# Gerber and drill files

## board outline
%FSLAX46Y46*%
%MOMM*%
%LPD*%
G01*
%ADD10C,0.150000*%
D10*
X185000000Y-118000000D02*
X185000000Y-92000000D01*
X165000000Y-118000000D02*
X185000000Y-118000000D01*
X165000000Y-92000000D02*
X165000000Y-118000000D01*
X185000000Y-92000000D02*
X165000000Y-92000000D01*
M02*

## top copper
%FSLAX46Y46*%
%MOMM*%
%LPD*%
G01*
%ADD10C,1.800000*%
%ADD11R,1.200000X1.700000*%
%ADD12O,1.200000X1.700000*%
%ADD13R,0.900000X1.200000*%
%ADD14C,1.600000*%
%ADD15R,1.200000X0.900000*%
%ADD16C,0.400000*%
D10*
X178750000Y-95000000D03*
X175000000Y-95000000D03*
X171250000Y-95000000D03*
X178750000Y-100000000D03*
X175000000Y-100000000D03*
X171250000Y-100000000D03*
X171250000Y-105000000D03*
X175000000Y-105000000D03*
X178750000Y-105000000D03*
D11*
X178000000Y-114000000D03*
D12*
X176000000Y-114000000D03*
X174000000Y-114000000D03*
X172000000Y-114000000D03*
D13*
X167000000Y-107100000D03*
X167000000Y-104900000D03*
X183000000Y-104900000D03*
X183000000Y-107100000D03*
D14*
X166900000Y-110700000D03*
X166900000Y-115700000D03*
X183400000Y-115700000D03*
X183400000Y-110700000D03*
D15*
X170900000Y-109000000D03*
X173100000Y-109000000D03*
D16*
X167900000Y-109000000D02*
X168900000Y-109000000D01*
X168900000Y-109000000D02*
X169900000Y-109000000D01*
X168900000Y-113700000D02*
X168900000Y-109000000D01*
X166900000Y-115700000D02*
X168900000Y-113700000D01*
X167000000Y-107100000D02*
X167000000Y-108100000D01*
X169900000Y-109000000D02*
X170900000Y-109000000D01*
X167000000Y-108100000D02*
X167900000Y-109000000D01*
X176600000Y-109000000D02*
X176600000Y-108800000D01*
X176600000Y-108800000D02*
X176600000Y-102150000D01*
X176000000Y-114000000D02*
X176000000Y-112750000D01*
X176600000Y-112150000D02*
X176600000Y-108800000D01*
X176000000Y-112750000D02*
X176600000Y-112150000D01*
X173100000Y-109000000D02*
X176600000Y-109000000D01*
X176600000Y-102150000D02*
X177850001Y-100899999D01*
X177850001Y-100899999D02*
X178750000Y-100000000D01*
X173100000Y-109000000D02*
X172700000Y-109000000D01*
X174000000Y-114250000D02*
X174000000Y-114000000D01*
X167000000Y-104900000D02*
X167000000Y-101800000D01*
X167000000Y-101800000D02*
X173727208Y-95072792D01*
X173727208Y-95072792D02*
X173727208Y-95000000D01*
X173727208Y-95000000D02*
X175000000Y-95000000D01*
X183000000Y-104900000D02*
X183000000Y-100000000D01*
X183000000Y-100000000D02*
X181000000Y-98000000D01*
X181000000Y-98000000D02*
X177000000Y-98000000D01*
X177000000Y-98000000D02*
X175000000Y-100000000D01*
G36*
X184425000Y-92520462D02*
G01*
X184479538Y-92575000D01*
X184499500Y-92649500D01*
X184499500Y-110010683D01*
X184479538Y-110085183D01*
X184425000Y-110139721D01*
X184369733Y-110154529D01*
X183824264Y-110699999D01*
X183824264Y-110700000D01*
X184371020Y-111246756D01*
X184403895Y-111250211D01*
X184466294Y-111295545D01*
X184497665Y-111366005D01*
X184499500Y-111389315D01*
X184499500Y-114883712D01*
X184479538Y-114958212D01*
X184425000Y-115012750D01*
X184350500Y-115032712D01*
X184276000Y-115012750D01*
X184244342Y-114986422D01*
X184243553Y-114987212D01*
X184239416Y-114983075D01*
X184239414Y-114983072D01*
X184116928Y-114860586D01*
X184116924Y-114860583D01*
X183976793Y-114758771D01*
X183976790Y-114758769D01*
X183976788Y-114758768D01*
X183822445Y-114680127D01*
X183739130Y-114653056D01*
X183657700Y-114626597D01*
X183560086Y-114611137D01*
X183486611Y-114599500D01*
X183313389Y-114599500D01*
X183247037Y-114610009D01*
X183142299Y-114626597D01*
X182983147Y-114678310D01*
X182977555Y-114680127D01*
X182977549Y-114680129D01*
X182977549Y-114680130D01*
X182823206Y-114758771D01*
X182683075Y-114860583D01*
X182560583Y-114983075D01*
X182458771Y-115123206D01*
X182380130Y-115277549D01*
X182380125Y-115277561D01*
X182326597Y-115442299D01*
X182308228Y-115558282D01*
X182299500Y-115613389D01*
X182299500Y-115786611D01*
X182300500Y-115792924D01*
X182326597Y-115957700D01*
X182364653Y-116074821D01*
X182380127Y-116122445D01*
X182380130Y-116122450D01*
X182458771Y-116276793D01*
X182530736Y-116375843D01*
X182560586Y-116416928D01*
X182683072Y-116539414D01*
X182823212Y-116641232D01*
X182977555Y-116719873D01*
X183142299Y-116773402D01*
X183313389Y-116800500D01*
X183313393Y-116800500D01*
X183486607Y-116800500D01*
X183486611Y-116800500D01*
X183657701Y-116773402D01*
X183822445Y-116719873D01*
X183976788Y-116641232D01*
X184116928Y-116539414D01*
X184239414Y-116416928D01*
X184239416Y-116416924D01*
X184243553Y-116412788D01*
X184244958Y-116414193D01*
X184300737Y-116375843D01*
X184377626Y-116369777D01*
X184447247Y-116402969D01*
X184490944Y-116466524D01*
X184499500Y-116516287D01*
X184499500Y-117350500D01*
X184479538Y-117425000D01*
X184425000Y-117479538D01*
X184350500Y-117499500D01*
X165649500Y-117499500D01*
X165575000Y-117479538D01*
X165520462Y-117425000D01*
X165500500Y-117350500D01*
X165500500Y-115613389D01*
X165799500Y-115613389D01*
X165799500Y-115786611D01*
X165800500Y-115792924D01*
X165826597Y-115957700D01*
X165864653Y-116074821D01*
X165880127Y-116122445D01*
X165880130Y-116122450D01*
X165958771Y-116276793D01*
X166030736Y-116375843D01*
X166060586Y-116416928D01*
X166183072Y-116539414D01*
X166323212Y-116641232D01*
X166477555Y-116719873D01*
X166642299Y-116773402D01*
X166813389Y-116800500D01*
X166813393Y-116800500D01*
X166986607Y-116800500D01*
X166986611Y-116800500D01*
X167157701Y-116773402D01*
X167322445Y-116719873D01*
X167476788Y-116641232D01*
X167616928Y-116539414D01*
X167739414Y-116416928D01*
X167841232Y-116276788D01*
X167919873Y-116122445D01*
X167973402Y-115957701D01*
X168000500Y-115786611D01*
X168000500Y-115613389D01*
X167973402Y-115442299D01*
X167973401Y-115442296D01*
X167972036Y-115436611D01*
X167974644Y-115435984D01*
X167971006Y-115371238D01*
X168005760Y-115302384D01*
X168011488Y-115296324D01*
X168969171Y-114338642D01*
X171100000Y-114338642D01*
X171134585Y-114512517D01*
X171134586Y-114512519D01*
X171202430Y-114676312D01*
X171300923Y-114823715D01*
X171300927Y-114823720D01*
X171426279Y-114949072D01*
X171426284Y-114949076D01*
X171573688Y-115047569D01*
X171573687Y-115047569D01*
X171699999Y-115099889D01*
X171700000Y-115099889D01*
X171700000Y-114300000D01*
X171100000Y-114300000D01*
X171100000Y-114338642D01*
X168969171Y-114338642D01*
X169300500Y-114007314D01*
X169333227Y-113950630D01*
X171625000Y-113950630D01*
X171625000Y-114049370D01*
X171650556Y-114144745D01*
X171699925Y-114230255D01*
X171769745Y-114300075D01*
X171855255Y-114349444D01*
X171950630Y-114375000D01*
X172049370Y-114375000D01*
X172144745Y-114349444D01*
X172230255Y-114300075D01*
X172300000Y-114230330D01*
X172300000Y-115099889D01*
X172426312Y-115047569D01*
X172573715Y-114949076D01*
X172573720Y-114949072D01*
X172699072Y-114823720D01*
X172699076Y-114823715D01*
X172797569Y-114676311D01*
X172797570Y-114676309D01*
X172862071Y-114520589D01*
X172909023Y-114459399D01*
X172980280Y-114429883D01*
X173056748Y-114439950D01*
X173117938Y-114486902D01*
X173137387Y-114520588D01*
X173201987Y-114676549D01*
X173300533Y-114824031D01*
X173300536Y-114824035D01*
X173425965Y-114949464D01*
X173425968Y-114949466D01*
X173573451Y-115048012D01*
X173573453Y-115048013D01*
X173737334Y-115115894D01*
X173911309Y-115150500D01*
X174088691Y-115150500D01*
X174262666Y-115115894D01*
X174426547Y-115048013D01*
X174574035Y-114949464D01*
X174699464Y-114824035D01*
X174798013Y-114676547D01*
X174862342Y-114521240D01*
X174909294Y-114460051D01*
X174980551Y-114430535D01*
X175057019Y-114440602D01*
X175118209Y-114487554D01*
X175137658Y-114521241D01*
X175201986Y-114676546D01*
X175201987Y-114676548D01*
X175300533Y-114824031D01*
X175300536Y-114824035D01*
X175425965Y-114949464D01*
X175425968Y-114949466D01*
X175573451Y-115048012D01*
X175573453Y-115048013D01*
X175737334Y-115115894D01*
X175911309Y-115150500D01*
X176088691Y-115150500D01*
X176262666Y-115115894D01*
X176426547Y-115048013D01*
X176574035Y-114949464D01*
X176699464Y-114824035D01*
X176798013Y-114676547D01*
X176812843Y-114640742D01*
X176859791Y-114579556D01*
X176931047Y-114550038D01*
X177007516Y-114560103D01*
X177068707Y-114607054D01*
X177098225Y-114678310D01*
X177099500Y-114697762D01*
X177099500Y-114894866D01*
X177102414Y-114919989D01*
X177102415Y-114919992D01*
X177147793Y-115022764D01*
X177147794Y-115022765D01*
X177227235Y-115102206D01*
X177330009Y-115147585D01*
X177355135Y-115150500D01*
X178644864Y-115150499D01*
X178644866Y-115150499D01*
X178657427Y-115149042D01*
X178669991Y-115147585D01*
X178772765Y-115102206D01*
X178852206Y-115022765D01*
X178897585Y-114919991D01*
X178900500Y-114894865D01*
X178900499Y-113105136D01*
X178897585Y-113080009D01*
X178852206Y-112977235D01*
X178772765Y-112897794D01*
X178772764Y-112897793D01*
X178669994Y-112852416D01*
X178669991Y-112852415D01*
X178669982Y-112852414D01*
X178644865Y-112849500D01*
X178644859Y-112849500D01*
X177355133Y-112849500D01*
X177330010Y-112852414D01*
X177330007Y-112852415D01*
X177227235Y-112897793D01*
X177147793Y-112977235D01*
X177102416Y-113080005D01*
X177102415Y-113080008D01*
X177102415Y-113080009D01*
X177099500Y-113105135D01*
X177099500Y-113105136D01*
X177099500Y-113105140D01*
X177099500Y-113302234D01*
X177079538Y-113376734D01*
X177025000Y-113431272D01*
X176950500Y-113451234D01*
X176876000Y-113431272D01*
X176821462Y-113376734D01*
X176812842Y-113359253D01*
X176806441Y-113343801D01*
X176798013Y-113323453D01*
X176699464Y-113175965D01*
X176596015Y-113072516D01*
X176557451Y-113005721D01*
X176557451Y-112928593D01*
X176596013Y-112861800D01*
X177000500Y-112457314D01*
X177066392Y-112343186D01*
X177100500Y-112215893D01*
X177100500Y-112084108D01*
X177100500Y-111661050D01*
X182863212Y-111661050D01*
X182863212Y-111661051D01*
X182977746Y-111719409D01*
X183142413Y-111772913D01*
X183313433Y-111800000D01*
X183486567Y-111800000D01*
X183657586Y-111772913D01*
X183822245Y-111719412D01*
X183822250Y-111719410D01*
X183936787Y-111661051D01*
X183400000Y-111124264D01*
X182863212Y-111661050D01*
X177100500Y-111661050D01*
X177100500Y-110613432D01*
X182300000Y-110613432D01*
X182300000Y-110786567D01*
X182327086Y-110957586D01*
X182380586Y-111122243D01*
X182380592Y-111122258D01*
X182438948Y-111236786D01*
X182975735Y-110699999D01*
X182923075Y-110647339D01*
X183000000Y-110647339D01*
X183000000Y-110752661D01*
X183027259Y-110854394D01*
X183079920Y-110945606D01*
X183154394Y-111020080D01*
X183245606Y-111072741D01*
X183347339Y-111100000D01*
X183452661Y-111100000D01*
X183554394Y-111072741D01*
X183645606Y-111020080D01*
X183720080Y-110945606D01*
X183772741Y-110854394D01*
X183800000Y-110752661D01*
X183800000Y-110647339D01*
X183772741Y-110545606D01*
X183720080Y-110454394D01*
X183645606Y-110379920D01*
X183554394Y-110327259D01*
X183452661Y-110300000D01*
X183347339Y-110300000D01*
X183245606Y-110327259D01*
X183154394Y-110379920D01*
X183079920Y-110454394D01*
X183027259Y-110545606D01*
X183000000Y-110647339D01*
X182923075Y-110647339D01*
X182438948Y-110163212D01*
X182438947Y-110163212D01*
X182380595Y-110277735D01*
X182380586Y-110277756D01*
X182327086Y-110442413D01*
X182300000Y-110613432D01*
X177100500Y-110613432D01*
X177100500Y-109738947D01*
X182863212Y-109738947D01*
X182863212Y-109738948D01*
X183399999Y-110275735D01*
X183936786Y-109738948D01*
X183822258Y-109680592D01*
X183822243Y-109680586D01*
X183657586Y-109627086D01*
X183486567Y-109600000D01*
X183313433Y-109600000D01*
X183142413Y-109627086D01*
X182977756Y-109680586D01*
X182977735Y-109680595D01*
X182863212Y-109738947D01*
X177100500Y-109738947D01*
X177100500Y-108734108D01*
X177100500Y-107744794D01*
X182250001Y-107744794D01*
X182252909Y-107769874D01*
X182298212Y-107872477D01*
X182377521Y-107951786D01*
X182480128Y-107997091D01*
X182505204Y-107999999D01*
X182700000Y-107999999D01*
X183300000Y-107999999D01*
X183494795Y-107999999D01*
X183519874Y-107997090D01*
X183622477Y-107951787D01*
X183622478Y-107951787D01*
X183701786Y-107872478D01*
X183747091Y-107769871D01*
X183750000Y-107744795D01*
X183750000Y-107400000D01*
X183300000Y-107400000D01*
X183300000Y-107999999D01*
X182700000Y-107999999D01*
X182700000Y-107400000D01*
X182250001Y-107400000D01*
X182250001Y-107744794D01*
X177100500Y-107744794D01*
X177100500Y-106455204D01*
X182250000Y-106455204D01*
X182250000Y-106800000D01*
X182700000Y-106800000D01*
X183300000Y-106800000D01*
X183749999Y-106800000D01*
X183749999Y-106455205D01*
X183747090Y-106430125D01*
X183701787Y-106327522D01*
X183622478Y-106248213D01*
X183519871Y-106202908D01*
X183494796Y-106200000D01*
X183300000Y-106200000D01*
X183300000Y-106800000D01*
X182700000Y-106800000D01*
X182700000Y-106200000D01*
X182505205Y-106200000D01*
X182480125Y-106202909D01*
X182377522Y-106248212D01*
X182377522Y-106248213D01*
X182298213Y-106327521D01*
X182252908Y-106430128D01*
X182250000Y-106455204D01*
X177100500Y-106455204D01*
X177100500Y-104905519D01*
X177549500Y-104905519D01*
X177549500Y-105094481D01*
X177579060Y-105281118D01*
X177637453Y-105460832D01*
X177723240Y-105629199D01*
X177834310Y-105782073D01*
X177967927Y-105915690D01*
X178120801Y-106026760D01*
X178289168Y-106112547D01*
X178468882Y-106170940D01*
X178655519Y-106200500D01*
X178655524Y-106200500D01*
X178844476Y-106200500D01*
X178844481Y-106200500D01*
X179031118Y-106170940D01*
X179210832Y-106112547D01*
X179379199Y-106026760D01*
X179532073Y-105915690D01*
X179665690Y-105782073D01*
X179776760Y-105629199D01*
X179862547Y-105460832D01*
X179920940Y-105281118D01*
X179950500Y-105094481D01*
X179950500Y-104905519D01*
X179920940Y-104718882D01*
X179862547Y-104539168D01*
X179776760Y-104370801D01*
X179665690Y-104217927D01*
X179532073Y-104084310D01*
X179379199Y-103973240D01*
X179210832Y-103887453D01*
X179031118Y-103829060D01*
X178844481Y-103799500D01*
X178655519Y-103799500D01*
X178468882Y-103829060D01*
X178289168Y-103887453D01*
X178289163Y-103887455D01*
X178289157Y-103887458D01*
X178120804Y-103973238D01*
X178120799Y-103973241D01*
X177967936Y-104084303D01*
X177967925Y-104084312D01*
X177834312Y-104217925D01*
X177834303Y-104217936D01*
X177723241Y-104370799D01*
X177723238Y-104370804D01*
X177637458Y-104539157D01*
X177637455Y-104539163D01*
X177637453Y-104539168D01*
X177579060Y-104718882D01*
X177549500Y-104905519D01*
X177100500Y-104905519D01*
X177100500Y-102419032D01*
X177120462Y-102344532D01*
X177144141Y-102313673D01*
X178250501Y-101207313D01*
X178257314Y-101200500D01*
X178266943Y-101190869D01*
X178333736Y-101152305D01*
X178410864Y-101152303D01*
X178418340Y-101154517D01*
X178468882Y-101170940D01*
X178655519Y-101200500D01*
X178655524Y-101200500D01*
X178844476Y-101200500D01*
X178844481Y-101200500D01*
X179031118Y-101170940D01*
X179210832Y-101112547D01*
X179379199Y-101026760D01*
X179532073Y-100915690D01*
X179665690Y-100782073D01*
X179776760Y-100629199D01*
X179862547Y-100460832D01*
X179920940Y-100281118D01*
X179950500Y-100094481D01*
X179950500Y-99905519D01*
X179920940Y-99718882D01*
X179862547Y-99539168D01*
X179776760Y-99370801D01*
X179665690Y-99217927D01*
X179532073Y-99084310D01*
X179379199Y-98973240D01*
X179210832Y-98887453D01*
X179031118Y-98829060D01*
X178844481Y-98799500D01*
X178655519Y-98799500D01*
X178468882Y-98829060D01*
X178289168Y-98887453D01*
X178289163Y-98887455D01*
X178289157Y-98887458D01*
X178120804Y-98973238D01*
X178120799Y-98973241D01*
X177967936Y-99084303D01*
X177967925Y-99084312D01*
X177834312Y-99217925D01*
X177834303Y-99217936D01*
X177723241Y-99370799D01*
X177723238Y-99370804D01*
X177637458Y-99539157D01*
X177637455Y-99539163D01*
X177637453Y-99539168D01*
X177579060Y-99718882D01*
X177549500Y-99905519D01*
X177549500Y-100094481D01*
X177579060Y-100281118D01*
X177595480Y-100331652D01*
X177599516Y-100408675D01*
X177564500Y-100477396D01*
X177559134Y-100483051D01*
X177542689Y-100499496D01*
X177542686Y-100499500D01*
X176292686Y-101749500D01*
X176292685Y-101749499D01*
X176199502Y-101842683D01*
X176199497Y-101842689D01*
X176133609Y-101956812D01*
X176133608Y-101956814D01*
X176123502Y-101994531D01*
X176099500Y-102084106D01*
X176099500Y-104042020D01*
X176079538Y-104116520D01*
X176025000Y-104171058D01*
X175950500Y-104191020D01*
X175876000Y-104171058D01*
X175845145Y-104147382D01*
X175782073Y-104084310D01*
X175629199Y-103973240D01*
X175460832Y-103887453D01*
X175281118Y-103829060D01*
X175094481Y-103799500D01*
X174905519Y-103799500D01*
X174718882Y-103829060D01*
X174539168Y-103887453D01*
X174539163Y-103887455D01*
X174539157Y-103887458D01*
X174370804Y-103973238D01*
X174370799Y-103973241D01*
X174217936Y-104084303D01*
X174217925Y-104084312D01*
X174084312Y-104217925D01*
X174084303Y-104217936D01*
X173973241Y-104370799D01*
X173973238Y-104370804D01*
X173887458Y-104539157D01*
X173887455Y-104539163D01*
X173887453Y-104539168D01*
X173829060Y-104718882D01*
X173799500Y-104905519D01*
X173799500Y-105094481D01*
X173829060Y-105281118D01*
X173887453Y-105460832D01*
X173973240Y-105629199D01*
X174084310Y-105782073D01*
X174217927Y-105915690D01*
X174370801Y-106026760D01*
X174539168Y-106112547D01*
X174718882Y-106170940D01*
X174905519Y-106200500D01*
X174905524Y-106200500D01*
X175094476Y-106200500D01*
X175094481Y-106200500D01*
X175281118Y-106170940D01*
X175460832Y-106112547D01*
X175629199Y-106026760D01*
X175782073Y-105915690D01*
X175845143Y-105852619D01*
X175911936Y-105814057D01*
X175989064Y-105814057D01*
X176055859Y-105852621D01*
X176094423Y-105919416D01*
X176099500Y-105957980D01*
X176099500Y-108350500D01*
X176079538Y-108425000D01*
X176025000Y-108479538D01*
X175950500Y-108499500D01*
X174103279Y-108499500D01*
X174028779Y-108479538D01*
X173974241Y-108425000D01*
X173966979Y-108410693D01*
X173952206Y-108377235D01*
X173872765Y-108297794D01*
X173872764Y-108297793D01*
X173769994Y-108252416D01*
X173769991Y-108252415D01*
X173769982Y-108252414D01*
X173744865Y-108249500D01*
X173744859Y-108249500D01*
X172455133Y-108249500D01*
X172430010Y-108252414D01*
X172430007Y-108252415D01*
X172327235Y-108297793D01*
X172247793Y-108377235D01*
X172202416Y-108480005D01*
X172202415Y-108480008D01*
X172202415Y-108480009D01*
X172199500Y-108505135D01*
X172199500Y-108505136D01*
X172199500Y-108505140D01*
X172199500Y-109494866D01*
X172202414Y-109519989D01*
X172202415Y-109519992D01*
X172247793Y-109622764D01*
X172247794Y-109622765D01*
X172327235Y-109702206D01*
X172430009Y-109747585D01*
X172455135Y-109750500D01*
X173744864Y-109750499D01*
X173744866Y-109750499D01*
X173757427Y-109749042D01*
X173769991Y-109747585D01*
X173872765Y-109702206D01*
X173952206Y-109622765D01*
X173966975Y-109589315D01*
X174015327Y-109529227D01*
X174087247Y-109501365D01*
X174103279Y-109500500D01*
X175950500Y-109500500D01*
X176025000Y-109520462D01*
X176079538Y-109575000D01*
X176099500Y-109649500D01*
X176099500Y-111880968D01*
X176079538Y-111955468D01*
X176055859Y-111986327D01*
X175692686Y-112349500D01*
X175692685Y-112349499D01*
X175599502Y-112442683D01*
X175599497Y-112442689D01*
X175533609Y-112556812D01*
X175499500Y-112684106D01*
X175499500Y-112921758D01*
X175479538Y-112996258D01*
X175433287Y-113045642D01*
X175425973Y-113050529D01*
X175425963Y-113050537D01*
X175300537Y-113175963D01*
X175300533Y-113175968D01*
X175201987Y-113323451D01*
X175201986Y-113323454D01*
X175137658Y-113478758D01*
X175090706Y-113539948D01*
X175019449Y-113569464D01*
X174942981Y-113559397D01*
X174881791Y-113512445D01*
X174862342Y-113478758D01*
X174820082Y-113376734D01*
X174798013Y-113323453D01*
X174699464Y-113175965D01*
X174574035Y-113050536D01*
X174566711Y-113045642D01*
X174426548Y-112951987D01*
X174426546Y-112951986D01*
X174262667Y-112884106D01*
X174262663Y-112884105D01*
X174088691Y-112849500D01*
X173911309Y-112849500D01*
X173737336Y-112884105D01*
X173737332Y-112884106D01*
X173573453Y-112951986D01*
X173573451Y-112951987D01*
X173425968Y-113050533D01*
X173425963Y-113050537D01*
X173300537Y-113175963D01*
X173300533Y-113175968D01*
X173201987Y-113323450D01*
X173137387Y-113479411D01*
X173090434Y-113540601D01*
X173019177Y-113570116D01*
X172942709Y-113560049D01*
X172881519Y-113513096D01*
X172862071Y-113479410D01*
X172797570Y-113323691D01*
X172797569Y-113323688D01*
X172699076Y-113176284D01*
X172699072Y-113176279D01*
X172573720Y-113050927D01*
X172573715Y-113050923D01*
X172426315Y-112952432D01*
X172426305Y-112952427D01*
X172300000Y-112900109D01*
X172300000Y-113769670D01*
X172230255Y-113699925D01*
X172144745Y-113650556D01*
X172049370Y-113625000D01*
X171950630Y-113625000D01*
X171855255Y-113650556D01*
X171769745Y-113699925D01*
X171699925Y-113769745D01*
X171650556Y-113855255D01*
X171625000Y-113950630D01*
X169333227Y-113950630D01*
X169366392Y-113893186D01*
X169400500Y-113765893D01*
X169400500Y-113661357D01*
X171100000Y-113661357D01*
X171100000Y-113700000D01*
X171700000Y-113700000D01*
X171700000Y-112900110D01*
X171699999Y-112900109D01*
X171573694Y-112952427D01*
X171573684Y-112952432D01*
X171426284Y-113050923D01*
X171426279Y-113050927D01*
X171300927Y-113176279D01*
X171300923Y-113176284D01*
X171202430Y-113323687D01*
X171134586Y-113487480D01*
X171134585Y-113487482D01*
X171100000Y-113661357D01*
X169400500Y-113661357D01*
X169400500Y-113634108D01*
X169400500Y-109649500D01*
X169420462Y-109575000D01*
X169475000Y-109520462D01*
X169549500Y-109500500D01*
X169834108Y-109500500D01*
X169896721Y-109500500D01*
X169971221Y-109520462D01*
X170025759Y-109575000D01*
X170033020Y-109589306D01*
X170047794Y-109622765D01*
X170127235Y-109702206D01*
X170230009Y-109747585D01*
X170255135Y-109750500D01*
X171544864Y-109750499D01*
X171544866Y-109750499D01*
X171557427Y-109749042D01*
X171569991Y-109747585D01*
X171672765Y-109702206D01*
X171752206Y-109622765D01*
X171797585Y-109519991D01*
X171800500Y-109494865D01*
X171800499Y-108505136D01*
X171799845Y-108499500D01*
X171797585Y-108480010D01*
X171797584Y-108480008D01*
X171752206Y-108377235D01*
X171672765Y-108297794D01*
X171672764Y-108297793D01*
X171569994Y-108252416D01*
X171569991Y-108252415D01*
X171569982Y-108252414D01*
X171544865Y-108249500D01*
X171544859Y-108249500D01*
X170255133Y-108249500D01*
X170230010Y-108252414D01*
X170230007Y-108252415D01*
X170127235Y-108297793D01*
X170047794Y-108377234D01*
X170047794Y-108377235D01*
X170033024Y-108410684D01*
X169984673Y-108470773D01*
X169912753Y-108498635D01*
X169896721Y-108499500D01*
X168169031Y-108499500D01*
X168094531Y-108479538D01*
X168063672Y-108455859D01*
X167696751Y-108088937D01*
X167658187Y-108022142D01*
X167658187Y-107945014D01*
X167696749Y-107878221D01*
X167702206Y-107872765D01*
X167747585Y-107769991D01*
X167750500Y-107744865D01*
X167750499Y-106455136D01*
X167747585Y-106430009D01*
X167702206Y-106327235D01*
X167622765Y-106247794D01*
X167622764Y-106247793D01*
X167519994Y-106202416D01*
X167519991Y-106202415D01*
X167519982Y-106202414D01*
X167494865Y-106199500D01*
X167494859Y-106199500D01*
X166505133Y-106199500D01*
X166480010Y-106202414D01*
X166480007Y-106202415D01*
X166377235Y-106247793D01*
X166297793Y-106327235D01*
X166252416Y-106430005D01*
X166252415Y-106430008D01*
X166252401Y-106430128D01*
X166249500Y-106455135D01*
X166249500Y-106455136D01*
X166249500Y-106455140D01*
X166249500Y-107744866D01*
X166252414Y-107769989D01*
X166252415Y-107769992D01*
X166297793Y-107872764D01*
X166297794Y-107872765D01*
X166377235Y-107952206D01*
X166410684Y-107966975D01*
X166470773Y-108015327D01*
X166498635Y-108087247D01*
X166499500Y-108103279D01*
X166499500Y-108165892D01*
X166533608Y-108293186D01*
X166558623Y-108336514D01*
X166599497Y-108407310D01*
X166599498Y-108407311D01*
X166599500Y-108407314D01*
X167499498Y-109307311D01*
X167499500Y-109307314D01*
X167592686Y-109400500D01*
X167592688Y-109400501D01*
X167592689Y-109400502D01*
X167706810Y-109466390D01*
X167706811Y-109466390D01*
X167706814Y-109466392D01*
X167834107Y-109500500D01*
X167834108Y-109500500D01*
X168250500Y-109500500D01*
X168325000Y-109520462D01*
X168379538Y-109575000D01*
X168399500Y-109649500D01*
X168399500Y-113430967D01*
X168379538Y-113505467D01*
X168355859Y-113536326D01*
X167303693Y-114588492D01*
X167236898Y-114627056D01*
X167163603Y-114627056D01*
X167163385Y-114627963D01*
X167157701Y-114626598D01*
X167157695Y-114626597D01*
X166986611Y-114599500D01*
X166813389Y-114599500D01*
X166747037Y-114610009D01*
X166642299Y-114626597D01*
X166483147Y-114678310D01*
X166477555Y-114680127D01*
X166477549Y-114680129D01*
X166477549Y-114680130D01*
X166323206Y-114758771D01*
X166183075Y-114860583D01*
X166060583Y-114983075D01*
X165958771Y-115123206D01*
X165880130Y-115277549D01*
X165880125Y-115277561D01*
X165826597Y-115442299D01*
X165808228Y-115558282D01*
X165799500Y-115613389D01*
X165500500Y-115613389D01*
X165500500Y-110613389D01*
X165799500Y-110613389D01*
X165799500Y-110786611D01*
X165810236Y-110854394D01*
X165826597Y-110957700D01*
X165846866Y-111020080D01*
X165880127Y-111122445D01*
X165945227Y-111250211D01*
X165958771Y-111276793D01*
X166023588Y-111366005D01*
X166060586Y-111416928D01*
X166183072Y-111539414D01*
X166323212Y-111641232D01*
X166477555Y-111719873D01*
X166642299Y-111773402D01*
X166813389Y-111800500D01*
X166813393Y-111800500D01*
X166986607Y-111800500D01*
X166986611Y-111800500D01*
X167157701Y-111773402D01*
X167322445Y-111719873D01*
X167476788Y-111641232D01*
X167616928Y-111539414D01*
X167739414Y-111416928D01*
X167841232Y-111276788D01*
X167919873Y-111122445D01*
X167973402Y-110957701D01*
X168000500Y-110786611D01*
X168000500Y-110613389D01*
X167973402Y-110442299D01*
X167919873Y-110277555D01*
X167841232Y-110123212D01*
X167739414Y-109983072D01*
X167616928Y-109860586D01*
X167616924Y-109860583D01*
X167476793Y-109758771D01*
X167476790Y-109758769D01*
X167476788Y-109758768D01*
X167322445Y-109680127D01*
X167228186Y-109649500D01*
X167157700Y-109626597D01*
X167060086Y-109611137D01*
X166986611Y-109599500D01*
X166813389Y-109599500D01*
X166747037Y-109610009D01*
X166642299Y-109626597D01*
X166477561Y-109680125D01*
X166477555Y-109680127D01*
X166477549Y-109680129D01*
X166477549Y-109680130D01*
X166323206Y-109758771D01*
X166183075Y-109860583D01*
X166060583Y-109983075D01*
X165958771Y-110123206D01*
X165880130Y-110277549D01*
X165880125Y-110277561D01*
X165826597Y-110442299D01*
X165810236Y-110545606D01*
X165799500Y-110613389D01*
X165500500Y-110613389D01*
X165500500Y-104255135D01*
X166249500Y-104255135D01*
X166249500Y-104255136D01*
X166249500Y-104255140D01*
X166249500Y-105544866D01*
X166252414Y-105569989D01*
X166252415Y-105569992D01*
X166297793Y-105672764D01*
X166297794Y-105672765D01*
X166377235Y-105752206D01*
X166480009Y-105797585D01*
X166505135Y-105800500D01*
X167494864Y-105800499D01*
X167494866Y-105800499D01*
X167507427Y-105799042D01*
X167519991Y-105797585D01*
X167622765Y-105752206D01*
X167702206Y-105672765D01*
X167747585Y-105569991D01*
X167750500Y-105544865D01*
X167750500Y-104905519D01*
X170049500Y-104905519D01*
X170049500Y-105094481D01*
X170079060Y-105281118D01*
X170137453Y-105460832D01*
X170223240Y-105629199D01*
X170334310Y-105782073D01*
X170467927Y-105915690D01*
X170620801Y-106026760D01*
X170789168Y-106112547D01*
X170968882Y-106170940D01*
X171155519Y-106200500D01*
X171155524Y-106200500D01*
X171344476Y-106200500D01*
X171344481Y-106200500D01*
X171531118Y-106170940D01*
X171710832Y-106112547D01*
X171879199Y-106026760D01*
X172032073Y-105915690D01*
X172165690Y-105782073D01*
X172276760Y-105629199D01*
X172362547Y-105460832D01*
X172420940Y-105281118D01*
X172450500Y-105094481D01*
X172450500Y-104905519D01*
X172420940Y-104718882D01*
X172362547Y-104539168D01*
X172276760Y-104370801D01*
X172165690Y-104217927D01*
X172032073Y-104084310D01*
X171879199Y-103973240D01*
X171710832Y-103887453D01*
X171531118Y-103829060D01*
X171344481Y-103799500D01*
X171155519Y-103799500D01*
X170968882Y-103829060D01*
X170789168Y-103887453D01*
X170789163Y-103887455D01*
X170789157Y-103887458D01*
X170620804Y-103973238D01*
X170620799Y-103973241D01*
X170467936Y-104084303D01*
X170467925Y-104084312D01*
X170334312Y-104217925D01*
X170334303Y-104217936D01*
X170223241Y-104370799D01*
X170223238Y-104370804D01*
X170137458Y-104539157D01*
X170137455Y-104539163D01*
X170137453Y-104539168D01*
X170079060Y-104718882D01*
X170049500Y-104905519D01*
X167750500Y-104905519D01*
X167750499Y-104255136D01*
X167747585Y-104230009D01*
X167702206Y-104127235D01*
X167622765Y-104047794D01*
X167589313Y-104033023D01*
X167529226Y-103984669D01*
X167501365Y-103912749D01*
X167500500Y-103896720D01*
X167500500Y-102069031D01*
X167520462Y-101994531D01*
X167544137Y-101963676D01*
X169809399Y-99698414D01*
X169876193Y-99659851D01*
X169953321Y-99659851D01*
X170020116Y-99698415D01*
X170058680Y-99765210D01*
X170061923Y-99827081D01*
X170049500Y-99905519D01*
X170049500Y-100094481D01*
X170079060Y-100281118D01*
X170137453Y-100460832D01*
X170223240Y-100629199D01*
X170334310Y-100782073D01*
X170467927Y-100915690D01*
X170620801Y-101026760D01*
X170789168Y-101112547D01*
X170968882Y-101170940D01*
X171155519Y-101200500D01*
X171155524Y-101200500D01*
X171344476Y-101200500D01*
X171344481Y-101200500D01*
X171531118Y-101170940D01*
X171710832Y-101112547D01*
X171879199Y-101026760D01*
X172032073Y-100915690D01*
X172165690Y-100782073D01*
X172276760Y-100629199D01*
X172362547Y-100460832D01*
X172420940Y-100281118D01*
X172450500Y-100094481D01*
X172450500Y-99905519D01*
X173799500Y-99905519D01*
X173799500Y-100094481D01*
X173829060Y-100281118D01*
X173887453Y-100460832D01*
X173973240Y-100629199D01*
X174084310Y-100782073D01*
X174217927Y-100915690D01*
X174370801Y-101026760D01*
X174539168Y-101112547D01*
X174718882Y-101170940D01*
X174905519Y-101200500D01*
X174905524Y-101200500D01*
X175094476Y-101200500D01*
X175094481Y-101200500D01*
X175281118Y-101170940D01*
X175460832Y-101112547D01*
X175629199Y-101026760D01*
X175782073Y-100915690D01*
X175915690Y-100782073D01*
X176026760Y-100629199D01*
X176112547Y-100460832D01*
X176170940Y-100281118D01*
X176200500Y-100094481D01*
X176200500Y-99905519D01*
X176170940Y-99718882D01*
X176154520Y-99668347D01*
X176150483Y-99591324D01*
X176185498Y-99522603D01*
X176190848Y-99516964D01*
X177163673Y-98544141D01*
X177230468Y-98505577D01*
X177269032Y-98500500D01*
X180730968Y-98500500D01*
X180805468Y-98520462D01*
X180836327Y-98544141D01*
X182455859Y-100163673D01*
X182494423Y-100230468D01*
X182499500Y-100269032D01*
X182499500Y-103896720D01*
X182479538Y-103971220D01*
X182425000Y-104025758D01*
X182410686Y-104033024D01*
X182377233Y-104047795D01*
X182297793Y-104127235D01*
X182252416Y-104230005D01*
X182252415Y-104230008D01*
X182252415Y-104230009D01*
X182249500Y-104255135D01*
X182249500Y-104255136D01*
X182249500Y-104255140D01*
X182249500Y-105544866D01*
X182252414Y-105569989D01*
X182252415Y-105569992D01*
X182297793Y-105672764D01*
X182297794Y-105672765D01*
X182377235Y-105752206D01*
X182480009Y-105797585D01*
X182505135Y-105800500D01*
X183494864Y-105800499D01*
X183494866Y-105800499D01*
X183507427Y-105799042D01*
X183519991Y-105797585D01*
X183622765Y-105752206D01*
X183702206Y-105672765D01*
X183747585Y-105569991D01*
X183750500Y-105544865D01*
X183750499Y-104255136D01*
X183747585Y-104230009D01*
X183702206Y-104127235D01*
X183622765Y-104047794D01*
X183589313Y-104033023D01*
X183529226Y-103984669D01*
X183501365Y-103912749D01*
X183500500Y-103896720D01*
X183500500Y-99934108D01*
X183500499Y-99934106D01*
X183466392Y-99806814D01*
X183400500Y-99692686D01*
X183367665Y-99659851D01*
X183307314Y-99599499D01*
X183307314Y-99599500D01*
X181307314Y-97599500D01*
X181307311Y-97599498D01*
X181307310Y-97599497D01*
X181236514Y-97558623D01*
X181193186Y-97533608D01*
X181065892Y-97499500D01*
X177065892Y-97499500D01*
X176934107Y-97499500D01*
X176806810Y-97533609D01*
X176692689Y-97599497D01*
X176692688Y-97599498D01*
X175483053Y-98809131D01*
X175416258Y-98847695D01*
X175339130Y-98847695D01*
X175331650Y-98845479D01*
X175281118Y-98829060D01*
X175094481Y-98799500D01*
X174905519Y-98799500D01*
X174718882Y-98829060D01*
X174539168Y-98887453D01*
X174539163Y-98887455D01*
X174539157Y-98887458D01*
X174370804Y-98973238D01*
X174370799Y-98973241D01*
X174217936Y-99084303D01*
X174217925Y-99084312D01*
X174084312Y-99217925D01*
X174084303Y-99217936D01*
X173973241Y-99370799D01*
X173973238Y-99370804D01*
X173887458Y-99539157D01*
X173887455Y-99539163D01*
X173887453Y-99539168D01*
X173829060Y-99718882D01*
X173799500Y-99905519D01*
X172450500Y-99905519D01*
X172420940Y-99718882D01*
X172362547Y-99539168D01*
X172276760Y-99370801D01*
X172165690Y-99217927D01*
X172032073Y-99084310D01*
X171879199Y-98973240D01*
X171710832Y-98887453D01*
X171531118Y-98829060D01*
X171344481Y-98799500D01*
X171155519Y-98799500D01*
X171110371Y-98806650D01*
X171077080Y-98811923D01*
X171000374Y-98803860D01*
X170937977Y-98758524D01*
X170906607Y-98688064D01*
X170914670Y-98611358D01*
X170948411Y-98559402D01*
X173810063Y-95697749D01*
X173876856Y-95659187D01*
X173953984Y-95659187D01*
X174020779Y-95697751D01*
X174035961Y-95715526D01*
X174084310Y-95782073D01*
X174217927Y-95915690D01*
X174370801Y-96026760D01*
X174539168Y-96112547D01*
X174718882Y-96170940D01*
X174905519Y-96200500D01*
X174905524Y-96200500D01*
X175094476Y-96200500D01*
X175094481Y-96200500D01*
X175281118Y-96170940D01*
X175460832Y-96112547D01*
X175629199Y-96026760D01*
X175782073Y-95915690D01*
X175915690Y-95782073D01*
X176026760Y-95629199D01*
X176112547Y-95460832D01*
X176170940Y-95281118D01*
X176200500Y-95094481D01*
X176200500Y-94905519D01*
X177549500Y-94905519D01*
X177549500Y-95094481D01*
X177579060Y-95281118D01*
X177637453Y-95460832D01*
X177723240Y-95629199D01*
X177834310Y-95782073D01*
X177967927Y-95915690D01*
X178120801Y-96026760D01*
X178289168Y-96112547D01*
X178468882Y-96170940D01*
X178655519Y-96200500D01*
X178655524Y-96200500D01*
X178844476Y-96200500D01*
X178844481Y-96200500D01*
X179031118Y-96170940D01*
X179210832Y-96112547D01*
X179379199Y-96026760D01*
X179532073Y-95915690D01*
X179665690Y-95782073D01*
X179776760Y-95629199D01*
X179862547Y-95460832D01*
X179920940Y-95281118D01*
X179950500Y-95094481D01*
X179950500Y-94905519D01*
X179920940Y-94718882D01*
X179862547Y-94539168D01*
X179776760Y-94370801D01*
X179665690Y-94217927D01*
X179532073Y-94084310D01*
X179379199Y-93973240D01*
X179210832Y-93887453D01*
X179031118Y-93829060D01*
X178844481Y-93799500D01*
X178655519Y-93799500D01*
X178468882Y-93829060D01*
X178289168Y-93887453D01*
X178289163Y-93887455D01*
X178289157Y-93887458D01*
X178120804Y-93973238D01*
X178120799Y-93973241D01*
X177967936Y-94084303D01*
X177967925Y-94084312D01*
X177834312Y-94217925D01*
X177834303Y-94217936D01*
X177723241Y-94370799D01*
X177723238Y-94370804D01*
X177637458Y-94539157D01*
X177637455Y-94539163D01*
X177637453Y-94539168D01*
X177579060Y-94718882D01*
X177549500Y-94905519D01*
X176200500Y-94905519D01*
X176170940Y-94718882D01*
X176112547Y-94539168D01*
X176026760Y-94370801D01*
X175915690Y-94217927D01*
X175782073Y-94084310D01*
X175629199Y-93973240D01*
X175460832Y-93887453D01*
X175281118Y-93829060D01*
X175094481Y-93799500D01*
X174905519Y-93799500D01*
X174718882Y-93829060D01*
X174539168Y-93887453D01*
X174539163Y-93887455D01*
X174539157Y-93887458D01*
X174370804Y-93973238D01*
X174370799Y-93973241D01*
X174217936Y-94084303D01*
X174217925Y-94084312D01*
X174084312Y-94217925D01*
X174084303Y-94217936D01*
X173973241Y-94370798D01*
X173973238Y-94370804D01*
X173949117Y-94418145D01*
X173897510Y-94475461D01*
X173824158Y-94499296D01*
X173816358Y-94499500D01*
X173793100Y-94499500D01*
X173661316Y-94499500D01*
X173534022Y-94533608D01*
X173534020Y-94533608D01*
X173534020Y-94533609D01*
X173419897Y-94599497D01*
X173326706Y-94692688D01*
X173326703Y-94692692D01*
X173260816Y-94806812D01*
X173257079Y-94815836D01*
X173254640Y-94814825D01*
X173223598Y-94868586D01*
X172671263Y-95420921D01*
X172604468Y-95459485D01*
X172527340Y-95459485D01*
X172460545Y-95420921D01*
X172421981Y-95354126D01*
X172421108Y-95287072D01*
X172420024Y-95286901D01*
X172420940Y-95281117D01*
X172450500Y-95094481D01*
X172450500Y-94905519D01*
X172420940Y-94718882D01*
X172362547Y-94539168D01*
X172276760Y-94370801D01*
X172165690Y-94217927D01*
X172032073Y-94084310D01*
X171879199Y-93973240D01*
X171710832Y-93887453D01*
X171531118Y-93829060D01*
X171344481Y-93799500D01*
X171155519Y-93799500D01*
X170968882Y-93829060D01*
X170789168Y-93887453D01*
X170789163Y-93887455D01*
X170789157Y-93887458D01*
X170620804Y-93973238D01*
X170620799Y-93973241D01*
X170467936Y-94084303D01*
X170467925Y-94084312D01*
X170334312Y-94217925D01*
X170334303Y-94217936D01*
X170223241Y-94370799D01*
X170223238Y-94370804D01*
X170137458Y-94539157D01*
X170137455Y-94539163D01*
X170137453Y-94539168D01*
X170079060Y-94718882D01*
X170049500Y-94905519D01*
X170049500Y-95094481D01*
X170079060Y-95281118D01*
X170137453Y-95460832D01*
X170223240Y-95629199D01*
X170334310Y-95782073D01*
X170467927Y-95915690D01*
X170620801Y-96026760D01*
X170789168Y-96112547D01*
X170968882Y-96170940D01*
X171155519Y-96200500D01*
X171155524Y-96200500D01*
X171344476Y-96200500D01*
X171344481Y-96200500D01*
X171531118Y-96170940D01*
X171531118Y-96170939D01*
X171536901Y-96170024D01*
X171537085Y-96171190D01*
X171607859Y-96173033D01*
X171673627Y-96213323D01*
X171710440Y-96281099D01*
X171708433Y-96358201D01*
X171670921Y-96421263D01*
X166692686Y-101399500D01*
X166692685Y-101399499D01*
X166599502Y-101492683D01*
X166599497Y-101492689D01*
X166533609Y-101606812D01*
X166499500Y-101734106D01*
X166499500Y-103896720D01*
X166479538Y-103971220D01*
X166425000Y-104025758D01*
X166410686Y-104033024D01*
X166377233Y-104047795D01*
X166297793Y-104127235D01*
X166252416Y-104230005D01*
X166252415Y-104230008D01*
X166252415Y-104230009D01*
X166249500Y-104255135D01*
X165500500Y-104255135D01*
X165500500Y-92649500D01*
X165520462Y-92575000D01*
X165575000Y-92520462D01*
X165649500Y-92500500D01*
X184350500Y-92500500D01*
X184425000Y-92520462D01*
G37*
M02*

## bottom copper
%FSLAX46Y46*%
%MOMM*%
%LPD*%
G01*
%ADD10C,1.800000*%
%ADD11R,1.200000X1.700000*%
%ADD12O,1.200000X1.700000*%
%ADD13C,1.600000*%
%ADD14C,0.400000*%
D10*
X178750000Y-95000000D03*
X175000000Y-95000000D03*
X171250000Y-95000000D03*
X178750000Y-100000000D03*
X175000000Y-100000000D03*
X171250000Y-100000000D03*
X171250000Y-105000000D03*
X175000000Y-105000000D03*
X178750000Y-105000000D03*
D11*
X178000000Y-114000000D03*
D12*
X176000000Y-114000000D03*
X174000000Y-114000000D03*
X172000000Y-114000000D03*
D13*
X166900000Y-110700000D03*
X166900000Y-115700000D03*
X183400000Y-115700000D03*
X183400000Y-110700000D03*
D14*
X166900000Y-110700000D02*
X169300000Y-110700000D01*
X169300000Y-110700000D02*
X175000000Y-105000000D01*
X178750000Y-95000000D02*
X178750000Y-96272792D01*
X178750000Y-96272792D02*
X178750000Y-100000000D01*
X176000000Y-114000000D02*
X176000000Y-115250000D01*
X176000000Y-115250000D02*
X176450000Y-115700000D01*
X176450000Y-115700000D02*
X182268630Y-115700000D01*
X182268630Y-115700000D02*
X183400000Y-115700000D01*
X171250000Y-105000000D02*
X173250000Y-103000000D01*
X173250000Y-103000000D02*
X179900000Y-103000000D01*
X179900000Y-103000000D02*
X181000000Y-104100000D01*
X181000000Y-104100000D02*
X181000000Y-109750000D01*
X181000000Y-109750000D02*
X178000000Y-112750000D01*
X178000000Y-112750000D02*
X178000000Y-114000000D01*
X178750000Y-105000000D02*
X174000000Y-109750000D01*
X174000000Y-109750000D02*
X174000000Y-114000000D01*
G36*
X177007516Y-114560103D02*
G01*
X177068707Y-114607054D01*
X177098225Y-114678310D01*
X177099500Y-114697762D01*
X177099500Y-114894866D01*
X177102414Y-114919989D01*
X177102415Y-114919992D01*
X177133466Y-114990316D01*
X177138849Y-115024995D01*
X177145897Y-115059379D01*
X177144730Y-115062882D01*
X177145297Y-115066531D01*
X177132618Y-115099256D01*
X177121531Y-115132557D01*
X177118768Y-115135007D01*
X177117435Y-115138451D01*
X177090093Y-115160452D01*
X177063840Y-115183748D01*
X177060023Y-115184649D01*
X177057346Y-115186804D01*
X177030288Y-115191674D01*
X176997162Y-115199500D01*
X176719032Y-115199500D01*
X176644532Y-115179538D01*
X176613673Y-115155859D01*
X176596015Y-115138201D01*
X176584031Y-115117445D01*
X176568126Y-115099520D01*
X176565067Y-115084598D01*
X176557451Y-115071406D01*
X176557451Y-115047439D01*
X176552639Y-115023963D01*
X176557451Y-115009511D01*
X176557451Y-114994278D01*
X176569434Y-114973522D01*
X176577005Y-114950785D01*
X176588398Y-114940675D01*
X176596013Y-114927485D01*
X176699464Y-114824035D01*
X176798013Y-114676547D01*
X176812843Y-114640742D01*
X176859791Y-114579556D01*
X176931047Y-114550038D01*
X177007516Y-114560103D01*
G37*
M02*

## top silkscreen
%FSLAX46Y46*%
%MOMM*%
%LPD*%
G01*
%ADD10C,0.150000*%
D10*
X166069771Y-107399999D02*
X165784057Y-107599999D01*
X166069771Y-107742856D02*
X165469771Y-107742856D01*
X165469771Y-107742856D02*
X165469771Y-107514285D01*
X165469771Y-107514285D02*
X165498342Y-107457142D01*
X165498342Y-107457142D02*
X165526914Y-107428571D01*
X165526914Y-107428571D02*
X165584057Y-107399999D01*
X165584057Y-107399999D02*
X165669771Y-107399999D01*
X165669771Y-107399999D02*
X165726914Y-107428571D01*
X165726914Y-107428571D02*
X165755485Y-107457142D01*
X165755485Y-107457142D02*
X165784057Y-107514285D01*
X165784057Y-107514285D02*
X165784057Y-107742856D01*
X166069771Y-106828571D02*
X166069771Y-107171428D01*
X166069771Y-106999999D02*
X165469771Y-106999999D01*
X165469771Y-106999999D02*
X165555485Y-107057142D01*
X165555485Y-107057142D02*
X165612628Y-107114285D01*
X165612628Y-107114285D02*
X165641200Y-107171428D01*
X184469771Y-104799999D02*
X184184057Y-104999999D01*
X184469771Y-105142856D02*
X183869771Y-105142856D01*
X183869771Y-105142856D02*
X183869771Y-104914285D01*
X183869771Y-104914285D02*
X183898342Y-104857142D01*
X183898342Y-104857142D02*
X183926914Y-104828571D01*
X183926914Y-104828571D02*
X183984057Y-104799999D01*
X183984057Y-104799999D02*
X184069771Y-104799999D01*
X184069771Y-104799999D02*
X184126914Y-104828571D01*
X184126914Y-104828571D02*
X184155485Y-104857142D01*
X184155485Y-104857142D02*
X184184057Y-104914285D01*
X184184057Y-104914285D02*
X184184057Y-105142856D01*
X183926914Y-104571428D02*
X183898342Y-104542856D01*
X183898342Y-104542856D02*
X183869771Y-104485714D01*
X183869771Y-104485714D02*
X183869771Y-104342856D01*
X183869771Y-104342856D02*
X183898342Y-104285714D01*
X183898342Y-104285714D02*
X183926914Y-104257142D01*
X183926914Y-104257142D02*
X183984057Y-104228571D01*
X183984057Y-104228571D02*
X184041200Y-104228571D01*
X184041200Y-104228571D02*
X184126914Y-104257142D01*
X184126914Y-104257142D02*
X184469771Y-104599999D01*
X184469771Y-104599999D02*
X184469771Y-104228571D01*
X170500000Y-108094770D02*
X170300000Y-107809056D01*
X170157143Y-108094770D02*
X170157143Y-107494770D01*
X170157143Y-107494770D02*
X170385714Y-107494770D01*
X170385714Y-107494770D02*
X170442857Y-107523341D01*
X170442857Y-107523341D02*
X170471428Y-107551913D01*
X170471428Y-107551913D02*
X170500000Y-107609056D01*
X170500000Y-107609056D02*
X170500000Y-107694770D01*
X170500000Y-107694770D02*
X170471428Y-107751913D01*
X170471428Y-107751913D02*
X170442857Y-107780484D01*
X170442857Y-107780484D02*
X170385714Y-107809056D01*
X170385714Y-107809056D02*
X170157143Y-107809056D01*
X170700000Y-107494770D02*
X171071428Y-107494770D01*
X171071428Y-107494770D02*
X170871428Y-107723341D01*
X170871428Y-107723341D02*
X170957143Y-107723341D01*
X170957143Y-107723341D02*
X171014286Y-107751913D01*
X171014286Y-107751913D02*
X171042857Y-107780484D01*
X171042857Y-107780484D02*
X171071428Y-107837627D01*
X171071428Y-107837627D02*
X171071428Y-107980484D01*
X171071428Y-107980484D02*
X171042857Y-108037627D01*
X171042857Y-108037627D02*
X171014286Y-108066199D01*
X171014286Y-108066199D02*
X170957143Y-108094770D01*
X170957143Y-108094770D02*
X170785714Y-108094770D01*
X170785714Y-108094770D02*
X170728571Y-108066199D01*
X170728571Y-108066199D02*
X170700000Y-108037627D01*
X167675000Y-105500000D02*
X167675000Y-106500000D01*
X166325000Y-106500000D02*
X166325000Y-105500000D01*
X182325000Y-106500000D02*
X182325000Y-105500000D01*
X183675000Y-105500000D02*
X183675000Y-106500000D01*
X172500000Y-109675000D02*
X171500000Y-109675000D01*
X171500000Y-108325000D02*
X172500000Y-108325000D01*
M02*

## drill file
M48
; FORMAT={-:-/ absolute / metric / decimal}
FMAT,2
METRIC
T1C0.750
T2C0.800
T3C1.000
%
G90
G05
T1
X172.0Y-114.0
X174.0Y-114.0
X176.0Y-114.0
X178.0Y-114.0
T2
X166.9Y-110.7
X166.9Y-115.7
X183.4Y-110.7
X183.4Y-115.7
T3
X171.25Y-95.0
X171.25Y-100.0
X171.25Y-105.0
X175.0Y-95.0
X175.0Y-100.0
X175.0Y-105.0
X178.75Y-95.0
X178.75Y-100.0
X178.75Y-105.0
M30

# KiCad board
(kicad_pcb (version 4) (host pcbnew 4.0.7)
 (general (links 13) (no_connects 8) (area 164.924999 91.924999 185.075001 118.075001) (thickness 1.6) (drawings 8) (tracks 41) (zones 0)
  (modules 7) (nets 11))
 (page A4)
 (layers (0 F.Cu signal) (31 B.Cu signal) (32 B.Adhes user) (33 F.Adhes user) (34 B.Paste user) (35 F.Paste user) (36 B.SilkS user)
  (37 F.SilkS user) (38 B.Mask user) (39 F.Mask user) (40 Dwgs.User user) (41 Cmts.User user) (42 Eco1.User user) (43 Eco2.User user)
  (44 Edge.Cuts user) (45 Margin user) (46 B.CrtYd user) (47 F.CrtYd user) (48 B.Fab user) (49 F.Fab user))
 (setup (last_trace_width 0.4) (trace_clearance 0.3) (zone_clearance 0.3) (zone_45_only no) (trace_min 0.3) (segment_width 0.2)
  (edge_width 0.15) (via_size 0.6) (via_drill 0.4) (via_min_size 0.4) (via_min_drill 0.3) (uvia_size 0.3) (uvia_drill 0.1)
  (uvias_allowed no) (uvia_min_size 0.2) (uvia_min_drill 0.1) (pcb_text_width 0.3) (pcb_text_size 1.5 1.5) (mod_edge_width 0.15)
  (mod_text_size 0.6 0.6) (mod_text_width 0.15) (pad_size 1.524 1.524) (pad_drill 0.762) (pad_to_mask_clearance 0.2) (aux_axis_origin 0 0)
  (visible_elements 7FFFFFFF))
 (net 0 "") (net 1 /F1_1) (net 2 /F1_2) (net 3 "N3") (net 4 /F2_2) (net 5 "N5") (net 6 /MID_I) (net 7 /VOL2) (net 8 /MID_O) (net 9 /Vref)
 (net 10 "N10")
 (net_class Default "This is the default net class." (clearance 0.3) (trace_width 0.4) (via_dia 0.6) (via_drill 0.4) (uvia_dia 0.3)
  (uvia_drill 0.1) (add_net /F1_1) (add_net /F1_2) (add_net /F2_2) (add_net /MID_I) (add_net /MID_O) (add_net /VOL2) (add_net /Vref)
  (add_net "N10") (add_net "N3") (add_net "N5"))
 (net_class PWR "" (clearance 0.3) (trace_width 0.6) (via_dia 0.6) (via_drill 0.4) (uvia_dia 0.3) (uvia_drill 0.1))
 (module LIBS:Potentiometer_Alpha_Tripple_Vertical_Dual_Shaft (layer B.Cu) (at 171.25 95 90)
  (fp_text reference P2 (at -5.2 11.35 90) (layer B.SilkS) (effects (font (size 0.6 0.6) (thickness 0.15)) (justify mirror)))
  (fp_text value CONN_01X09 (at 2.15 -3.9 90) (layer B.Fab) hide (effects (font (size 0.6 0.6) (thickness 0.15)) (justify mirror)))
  (pad 3 thru_hole circle (at 0 7.5 90) (size 1.8 1.8) (drill 1) (layers *.Cu *.Mask) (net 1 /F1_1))
  (pad 2 thru_hole circle (at 0 3.75 90) (size 1.8 1.8) (drill 1) (layers *.Cu *.Mask) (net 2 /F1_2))
  (pad 1 thru_hole circle (at 0 0 90) (size 1.8 1.8) (drill 1) (layers *.Cu *.Mask) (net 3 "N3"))
  (pad 6 thru_hole circle (at -5 7.5 90) (size 1.8 1.8) (drill 1) (layers *.Cu *.Mask) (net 1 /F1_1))
  (pad 5 thru_hole circle (at -5 3.75 90) (size 1.8 1.8) (drill 1) (layers *.Cu *.Mask) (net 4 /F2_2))
  (pad 4 thru_hole circle (at -5 0 90) (size 1.8 1.8) (drill 1) (layers *.Cu *.Mask) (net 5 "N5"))
  (pad 7 thru_hole circle (at -10 0 90) (size 1.8 1.8) (drill 1) (layers *.Cu *.Mask) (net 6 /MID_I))
  (pad 8 thru_hole circle (at -10 3.75 90) (size 1.8 1.8) (drill 1) (layers *.Cu *.Mask) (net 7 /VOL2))
  (pad 9 thru_hole circle (at -10 7.5 90) (size 1.8 1.8) (drill 1) (layers *.Cu *.Mask) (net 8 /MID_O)))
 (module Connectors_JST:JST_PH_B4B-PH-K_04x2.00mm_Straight (layer B.Cu) (at 178 114 180)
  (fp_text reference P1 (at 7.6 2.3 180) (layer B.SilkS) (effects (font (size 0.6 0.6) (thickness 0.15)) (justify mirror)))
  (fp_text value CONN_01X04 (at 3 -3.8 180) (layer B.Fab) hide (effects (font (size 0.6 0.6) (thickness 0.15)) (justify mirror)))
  (pad 1 thru_hole rect (at 0 0 180) (size 1.2 1.7) (drill 0.75) (layers *.Cu *.Mask) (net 6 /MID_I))
  (pad 2 thru_hole oval (at 2 0 180) (size 1.2 1.7) (drill 0.75) (layers *.Cu *.Mask) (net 1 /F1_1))
  (pad 3 thru_hole oval (at 4 0 180) (size 1.2 1.7) (drill 0.75) (layers *.Cu *.Mask) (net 8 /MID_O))
  (pad 4 thru_hole oval (at 6 0 180) (size 1.2 1.7) (drill 0.75) (layers *.Cu *.Mask) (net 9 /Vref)))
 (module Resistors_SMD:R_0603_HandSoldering (layer F.Cu) (at 167 106 90)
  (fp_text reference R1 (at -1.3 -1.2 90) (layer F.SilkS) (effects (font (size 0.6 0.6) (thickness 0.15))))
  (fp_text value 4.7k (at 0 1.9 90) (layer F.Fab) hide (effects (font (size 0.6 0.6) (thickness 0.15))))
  (fp_line (start 0.5 0.675) (end -0.5 0.675) (layer F.SilkS) (width 0.15))
  (fp_line (start -0.5 -0.675) (end 0.5 -0.675) (layer F.SilkS) (width 0.15))
  (pad 1 smd rect (at -1.1 0 90) (size 1.2 0.9) (layers F.Cu F.Paste F.Mask) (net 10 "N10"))
  (pad 2 smd rect (at 1.1 0 90) (size 1.2 0.9) (layers F.Cu F.Paste F.Mask) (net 2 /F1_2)))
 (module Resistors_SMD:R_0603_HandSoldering (layer F.Cu) (at 183 106 270)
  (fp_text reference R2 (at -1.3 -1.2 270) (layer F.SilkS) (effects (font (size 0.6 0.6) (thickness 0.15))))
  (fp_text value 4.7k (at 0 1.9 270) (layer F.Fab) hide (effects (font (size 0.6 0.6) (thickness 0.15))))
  (fp_line (start 0.5 0.675) (end -0.5 0.675) (layer F.SilkS) (width 0.15))
  (fp_line (start -0.5 -0.675) (end 0.5 -0.675) (layer F.SilkS) (width 0.15))
  (pad 1 smd rect (at -1.1 0 270) (size 1.2 0.9) (layers F.Cu F.Paste F.Mask) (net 4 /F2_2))
  (pad 2 smd rect (at 1.1 0 270) (size 1.2 0.9) (layers F.Cu F.Paste F.Mask) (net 9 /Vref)))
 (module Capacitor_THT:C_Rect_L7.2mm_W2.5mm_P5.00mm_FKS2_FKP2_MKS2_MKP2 (layer B.Cu) (at 166.9 110.7 270)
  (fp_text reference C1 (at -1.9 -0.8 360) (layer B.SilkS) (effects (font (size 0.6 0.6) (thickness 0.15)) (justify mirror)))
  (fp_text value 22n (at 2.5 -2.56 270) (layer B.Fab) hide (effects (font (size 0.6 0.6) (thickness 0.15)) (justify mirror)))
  (pad 1 thru_hole circle (at 0 0 270) (size 1.6 1.6) (drill 0.8) (layers *.Cu *.Mask) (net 7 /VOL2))
  (pad 2 thru_hole circle (at 5 0 270) (size 1.6 1.6) (drill 0.8) (layers *.Cu *.Mask) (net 10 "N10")))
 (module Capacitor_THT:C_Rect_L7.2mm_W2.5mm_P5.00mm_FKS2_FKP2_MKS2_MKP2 (layer B.Cu) (at 183.4 115.7 90)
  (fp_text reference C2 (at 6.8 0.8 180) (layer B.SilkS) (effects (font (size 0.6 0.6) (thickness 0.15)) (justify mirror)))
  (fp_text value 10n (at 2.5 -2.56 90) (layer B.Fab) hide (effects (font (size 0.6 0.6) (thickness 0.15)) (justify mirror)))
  (pad 1 thru_hole circle (at 0 0 90) (size 1.6 1.6) (drill 0.8) (layers *.Cu *.Mask) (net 1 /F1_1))
  (pad 2 thru_hole circle (at 5 0 90) (size 1.6 1.6) (drill 0.8) (layers *.Cu *.Mask) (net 9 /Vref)))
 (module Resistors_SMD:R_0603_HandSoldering (layer F.Cu) (at 172 109)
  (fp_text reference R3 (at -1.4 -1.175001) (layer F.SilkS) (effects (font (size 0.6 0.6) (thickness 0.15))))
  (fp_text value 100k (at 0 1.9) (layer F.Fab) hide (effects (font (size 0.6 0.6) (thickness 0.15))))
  (fp_line (start 0.5 0.675) (end -0.5 0.675) (layer F.SilkS) (width 0.15))
  (fp_line (start -0.5 -0.675) (end 0.5 -0.675) (layer F.SilkS) (width 0.15))
  (pad 1 smd rect (at -1.1 0) (size 1.2 0.9) (layers F.Cu F.Paste F.Mask) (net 10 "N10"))
  (pad 2 smd rect (at 1.1 0) (size 1.2 0.9) (layers F.Cu F.Paste F.Mask) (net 1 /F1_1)))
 (gr_line (start 185 118) (end 185 92) (layer Edge.Cuts) (width 0.15))
 (gr_line (start 165 118) (end 185 118) (layer Edge.Cuts) (width 0.15))
 (gr_line (start 165 92) (end 165 118) (layer Edge.Cuts) (width 0.15))
 (gr_line (start 185 92) (end 165 92) (layer Edge.Cuts) (width 0.15))
 (segment (start 166.9 110.7) (end 169.3 110.7) (width 0.4) (layer B.Cu) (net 7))
 (segment (start 169.3 110.7) (end 175 105) (width 0.4) (layer B.Cu) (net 7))
 (segment (start 167.9 109) (end 168.9 109) (width 0.4) (layer F.Cu) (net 10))
 (segment (start 168.9 109) (end 169.9 109) (width 0.4) (layer F.Cu) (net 10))
 (segment (start 168.9 113.7) (end 168.9 109) (width 0.4) (layer F.Cu) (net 10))
 (segment (start 166.9 115.7) (end 168.9 113.7) (width 0.4) (layer F.Cu) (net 10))
 (segment (start 167 107.1) (end 167 108.1) (width 0.4) (layer F.Cu) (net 10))
 (segment (start 169.9 109) (end 170.9 109) (width 0.4) (layer F.Cu) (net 10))
 (segment (start 167 108.1) (end 167.9 109) (width 0.4) (layer F.Cu) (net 10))
 (segment (start 178.75 95) (end 178.75 96.272792) (width 0.4) (layer B.Cu) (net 1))
 (segment (start 178.75 96.272792) (end 178.75 100) (width 0.4) (layer B.Cu) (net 1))
 (segment (start 176.6 109) (end 176.6 108.8) (width 0.4) (layer F.Cu) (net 1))
 (segment (start 176.6 108.8) (end 176.6 102.15) (width 0.4) (layer F.Cu) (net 1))
 (segment (start 176 114) (end 176 112.75) (width 0.4) (layer F.Cu) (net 1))
 (segment (start 176.6 112.15) (end 176.6 108.8) (width 0.4) (layer F.Cu) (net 1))
 (segment (start 176 112.75) (end 176.6 112.15) (width 0.4) (layer F.Cu) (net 1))
 (segment (start 173.1 109) (end 176.6 109) (width 0.4) (layer F.Cu) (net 1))
 (segment (start 176.6 102.15) (end 177.850001 100.899999) (width 0.4) (layer F.Cu) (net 1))
 (segment (start 177.850001 100.899999) (end 178.75 100) (width 0.4) (layer F.Cu) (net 1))
 (segment (start 173.1 109) (end 172.7 109) (width 0.4) (layer F.Cu) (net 1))
 (segment (start 176 114) (end 176 115.25) (width 0.4) (layer B.Cu) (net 1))
 (segment (start 176 115.25) (end 176.45 115.7) (width 0.4) (layer B.Cu) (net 1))
 (segment (start 176.45 115.7) (end 182.26863 115.7) (width 0.4) (layer B.Cu) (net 1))
 (segment (start 182.26863 115.7) (end 183.4 115.7) (width 0.4) (layer B.Cu) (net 1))
 (segment (start 171.25 105) (end 173.25 103) (width 0.4) (layer B.Cu) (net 6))
 (segment (start 173.25 103) (end 179.9 103) (width 0.4) (layer B.Cu) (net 6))
 (segment (start 179.9 103) (end 181 104.1) (width 0.4) (layer B.Cu) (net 6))
 (segment (start 181 104.1) (end 181 109.75) (width 0.4) (layer B.Cu) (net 6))
 (segment (start 181 109.75) (end 178 112.75) (width 0.4) (layer B.Cu) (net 6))
 (segment (start 178 112.75) (end 178 114) (width 0.4) (layer B.Cu) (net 6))
 (segment (start 178.75 105) (end 174 109.75) (width 0.4) (layer B.Cu) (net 8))
 (segment (start 174 109.75) (end 174 114) (width 0.4) (layer B.Cu) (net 8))
 (segment (start 174 114.25) (end 174 114) (width 0.4) (layer F.Cu) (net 8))
 (segment (start 167 104.9) (end 167 101.8) (width 0.4) (layer F.Cu) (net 2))
 (segment (start 167 101.8) (end 173.727208 95.072792) (width 0.4) (layer F.Cu) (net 2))
 (segment (start 173.727208 95.072792) (end 173.727208 95) (width 0.4) (layer F.Cu) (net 2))
 (segment (start 173.727208 95) (end 175 95) (width 0.4) (layer F.Cu) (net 2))
 (segment (start 183 104.9) (end 183 100) (width 0.4) (layer F.Cu) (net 4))
 (segment (start 183 100) (end 181 98) (width 0.4) (layer F.Cu) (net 4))
 (segment (start 181 98) (end 177 98) (width 0.4) (layer F.Cu) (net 4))
 (segment (start 177 98) (end 175 100) (width 0.4) (layer F.Cu) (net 4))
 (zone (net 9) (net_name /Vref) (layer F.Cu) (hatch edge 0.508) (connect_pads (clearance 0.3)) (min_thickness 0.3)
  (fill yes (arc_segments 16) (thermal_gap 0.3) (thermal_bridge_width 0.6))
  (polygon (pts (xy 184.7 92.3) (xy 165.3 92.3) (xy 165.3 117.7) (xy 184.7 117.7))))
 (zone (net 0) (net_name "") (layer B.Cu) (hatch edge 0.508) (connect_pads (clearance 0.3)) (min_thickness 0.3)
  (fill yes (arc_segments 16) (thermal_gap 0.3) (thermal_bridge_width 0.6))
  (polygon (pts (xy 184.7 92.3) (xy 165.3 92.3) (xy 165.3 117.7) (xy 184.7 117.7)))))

